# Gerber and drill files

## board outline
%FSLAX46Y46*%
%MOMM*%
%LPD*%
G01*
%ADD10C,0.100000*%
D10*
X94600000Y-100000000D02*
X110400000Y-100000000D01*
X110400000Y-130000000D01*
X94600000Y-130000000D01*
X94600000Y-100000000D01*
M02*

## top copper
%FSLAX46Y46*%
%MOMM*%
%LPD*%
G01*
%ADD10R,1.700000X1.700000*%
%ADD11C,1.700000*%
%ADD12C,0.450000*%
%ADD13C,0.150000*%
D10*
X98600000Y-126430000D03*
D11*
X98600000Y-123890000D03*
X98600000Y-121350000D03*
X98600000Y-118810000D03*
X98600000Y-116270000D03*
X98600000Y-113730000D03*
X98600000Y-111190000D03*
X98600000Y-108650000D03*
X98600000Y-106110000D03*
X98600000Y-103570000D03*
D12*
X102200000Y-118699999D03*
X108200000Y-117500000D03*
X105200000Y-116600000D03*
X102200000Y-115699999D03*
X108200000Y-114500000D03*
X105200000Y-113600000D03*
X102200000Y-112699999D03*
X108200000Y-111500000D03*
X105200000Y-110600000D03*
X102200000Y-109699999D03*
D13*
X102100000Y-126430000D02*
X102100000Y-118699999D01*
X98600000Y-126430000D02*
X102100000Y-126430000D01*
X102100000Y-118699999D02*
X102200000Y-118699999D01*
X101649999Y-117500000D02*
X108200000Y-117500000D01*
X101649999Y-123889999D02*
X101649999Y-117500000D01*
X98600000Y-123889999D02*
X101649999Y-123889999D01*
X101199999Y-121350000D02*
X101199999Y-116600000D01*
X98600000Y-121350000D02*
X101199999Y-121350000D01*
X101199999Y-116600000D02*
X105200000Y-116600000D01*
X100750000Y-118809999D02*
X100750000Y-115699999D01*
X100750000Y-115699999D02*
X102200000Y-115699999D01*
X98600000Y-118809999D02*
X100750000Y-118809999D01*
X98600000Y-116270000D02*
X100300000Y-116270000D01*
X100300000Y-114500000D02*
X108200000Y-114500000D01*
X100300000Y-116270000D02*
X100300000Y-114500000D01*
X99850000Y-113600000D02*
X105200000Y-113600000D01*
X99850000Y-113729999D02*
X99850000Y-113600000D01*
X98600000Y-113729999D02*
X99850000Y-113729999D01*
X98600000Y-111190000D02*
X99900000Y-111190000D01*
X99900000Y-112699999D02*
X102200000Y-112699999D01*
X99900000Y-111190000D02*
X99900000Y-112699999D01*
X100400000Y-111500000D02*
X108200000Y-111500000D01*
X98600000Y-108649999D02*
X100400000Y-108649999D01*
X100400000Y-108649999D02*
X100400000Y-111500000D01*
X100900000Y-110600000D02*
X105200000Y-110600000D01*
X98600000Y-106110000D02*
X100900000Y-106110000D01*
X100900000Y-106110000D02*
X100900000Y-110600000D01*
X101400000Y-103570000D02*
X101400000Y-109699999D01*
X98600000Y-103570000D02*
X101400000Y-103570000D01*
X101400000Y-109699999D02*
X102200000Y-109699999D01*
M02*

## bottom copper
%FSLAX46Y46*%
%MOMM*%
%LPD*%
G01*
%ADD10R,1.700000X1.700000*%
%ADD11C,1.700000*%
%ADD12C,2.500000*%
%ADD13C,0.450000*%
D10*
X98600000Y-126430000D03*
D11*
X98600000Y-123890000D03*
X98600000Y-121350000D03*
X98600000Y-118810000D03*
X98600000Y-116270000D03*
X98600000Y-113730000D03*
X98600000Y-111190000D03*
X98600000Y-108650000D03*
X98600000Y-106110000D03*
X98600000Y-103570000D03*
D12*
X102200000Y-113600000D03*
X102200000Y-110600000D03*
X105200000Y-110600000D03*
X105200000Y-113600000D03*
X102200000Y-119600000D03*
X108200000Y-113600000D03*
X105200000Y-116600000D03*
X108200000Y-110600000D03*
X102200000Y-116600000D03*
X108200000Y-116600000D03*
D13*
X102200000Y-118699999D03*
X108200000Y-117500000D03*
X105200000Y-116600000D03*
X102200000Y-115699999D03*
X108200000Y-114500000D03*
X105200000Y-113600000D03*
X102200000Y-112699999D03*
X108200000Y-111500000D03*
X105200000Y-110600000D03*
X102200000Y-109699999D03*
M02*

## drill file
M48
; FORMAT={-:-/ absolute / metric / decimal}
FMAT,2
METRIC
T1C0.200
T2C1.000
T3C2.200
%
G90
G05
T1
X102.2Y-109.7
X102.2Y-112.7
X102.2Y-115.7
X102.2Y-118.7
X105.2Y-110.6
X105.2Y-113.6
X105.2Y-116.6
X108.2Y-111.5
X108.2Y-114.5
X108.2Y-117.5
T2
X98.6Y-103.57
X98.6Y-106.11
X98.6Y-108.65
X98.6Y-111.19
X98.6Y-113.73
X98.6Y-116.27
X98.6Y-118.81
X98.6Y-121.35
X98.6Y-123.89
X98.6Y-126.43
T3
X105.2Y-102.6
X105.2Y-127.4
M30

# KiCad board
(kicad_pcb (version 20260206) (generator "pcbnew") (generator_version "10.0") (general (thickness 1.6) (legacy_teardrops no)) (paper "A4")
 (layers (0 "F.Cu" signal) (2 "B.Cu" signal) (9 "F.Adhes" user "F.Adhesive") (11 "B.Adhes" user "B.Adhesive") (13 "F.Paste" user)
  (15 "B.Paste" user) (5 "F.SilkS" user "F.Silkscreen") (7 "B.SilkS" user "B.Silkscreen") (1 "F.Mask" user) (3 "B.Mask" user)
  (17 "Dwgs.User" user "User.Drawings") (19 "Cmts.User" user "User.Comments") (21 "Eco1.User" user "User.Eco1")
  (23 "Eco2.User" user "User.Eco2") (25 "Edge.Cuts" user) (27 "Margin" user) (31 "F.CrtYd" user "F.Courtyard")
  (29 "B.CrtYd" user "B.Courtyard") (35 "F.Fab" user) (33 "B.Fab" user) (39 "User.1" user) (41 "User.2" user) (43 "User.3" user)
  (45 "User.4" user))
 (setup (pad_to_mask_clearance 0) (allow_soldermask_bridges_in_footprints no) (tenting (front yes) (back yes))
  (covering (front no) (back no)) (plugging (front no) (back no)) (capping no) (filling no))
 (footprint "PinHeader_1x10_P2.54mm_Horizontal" (layer "F.Cu") (at 98.6 126.43 180)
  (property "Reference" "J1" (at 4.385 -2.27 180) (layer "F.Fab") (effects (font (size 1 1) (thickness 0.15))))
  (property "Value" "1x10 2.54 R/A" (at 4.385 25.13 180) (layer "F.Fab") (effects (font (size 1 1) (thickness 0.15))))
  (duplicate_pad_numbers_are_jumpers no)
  (pad "1" thru_hole rect (at 0 0 180) (size 1.7 1.7) (drill 1) (layers "*.Cu" "*.Mask") (remove_unused_layers no) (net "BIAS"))
  (pad "2" thru_hole circle (at 0 2.54 180) (size 1.7 1.7) (drill 1) (layers "*.Cu" "*.Mask") (remove_unused_layers no) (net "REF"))
  (pad "3" thru_hole circle (at 0 5.08 180) (size 1.7 1.7) (drill 1) (layers "*.Cu" "*.Mask") (remove_unused_layers no) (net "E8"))
  (pad "4" thru_hole circle (at 0 7.62 180) (size 1.7 1.7) (drill 1) (layers "*.Cu" "*.Mask") (remove_unused_layers no) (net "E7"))
  (pad "5" thru_hole circle (at 0 10.16 180) (size 1.7 1.7) (drill 1) (layers "*.Cu" "*.Mask") (remove_unused_layers no) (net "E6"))
  (pad "6" thru_hole circle (at 0 12.7 180) (size 1.7 1.7) (drill 1) (layers "*.Cu" "*.Mask") (remove_unused_layers no) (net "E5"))
  (pad "7" thru_hole circle (at 0 15.24 180) (size 1.7 1.7) (drill 1) (layers "*.Cu" "*.Mask") (remove_unused_layers no) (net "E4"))
  (pad "8" thru_hole circle (at 0 17.78 180) (size 1.7 1.7) (drill 1) (layers "*.Cu" "*.Mask") (remove_unused_layers no) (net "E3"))
  (pad "9" thru_hole circle (at 0 20.32 180) (size 1.7 1.7) (drill 1) (layers "*.Cu" "*.Mask") (remove_unused_layers no) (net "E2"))
  (pad "10" thru_hole circle (at 0 22.86 180) (size 1.7 1.7) (drill 1) (layers "*.Cu" "*.Mask") (remove_unused_layers no) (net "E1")))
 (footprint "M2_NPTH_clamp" (layer "F.Cu") (at 105.2 102.6)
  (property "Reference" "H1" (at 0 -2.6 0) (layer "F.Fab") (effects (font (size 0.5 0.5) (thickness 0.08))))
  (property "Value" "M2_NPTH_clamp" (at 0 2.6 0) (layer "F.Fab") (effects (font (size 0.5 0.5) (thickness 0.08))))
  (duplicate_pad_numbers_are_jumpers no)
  (pad "" np_thru_hole circle (at 0 0) (size 2.2 2.2) (drill 2.2) (layers "*.Cu" "*.Mask")))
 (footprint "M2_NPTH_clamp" (layer "F.Cu") (at 105.2 127.4)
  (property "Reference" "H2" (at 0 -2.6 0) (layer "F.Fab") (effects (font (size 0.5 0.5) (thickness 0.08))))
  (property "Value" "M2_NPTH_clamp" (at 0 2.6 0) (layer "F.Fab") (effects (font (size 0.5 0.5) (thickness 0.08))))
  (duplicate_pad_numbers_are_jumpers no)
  (pad "" np_thru_hole circle (at 0 0) (size 2.2 2.2) (drill 2.2) (layers "*.Cu" "*.Mask")))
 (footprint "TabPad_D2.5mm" (layer "B.Cu") (at 102.2 113.6 180)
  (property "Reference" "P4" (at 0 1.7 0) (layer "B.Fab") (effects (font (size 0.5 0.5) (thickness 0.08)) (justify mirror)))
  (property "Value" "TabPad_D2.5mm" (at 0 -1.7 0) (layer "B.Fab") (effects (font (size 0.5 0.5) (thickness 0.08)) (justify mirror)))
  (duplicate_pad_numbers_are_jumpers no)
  (pad "1" smd circle (at 0 0 180) (size 2.5 2.5) (layers "B.Cu" "B.Mask") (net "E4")))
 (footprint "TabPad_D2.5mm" (layer "B.Cu") (at 102.2 110.6 180)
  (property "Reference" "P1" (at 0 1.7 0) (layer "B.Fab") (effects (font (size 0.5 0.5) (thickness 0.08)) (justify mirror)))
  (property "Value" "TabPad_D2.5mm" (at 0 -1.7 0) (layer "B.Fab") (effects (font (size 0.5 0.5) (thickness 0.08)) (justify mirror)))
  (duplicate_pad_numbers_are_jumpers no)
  (pad "1" smd circle (at 0 0 180) (size 2.5 2.5) (layers "B.Cu" "B.Mask") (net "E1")))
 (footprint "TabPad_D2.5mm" (layer "B.Cu") (at 105.2 110.6 180)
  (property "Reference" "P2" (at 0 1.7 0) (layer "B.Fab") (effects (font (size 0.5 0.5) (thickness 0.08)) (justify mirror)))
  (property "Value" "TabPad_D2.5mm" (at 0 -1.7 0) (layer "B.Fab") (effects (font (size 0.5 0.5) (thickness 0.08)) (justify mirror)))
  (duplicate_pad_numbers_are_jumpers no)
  (pad "1" smd circle (at 0 0 180) (size 2.5 2.5) (layers "B.Cu" "B.Mask") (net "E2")))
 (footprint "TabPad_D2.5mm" (layer "B.Cu") (at 105.2 113.6 180)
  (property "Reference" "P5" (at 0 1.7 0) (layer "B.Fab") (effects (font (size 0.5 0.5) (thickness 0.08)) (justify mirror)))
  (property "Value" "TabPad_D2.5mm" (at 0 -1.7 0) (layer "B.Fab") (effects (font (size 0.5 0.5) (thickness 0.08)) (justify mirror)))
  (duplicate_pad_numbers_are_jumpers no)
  (pad "1" smd circle (at 0 0 180) (size 2.5 2.5) (layers "B.Cu" "B.Mask") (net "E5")))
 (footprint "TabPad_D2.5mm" (layer "B.Cu") (at 102.2 119.6 180)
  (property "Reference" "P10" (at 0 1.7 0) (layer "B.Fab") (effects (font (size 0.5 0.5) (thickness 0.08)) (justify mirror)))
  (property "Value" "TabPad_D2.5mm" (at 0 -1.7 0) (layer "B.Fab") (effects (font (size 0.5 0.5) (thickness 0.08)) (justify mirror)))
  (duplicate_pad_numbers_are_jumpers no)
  (pad "1" smd circle (at 0 0 180) (size 2.5 2.5) (layers "B.Cu" "B.Mask") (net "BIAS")))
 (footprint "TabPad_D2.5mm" (layer "B.Cu") (at 108.2 113.6 180)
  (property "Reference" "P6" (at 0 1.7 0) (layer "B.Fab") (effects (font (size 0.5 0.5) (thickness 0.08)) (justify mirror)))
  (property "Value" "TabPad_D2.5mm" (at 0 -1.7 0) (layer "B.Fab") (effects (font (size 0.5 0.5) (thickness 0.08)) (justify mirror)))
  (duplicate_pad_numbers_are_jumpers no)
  (pad "1" smd circle (at 0 0 180) (size 2.5 2.5) (layers "B.Cu" "B.Mask") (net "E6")))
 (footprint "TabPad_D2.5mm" (layer "B.Cu") (at 105.2 116.6 180)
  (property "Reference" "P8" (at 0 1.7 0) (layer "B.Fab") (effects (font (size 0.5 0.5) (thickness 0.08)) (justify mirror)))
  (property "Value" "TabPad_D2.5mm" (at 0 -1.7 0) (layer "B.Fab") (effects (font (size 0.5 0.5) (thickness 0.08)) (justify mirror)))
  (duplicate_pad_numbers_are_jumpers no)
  (pad "1" smd circle (at 0 0 180) (size 2.5 2.5) (layers "B.Cu" "B.Mask") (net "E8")))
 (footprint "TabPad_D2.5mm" (layer "B.Cu") (at 108.2 110.6 180)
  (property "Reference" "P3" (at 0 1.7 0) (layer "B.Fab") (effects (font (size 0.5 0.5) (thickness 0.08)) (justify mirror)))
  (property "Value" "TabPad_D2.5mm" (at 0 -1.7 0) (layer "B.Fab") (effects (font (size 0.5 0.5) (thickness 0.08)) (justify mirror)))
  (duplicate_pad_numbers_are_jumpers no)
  (pad "1" smd circle (at 0 0 180) (size 2.5 2.5) (layers "B.Cu" "B.Mask") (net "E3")))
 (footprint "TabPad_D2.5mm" (layer "B.Cu") (at 102.2 116.6 180)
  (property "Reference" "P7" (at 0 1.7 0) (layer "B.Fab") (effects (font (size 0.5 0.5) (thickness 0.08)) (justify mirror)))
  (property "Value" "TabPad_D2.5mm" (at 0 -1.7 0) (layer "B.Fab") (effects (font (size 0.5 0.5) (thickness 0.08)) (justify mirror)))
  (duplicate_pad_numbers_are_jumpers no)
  (pad "1" smd circle (at 0 0 180) (size 2.5 2.5) (layers "B.Cu" "B.Mask") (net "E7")))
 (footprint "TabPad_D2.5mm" (layer "B.Cu") (at 108.2 116.6 180)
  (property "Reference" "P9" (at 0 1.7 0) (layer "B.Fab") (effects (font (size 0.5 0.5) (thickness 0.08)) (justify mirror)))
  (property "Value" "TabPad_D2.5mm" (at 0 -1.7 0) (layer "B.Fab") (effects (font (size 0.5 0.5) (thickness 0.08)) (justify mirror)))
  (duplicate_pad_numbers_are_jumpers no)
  (pad "1" smd circle (at 0 0 180) (size 2.5 2.5) (layers "B.Cu" "B.Mask") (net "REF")))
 (gr_rect (start 94.6 100) (end 110.4 130) (stroke (width 0.1) (type default)) (fill no) (layer "Edge.Cuts"))
 (segment (start 102.1 126.43) (end 102.1 118.699999) (width 0.15) (layer "F.Cu") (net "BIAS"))
 (segment (start 98.6 126.43) (end 102.1 126.43) (width 0.15) (layer "F.Cu") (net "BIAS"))
 (segment (start 102.1 118.699999) (end 102.2 118.699999) (width 0.15) (layer "F.Cu") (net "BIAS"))
 (via (at 102.2 118.699999) (size 0.45) (drill 0.2) (layers "F.Cu" "B.Cu") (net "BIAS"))
 (segment (start 101.649999 117.5) (end 108.2 117.5) (width 0.15) (layer "F.Cu") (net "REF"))
 (segment (start 101.649999 123.889999) (end 101.649999 117.5) (width 0.15) (layer "F.Cu") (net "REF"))
 (segment (start 98.6 123.889999) (end 101.649999 123.889999) (width 0.15) (layer "F.Cu") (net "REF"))
 (via (at 108.2 117.5) (size 0.45) (drill 0.2) (layers "F.Cu" "B.Cu") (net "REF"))
 (segment (start 101.199999 121.35) (end 101.199999 116.6) (width 0.15) (layer "F.Cu") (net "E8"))
 (segment (start 98.6 121.35) (end 101.199999 121.35) (width 0.15) (layer "F.Cu") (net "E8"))
 (segment (start 101.199999 116.6) (end 105.2 116.6) (width 0.15) (layer "F.Cu") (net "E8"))
 (via (at 105.2 116.6) (size 0.45) (drill 0.2) (layers "F.Cu" "B.Cu") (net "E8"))
 (segment (start 100.75 118.809999) (end 100.75 115.699999) (width 0.15) (layer "F.Cu") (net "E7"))
 (segment (start 100.75 115.699999) (end 102.2 115.699999) (width 0.15) (layer "F.Cu") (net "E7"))
 (segment (start 98.6 118.809999) (end 100.75 118.809999) (width 0.15) (layer "F.Cu") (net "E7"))
 (via (at 102.2 115.699999) (size 0.45) (drill 0.2) (layers "F.Cu" "B.Cu") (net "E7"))
 (segment (start 98.6 116.27) (end 100.3 116.27) (width 0.15) (layer "F.Cu") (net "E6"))
 (segment (start 100.3 114.5) (end 108.2 114.5) (width 0.15) (layer "F.Cu") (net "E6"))
 (segment (start 100.3 116.27) (end 100.3 114.5) (width 0.15) (layer "F.Cu") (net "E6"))
 (via (at 108.2 114.5) (size 0.45) (drill 0.2) (layers "F.Cu" "B.Cu") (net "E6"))
 (segment (start 99.85 113.6) (end 105.2 113.6) (width 0.15) (layer "F.Cu") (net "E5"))
 (segment (start 99.85 113.729999) (end 99.85 113.6) (width 0.15) (layer "F.Cu") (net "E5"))
 (segment (start 98.6 113.729999) (end 99.85 113.729999) (width 0.15) (layer "F.Cu") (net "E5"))
 (via (at 105.2 113.6) (size 0.45) (drill 0.2) (layers "F.Cu" "B.Cu") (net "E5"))
 (segment (start 98.6 111.19) (end 99.9 111.19) (width 0.15) (layer "F.Cu") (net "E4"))
 (segment (start 99.9 112.699999) (end 102.2 112.699999) (width 0.15) (layer "F.Cu") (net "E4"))
 (segment (start 99.9 111.19) (end 99.9 112.699999) (width 0.15) (layer "F.Cu") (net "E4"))
 (via (at 102.2 112.699999) (size 0.45) (drill 0.2) (layers "F.Cu" "B.Cu") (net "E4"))
 (segment (start 100.4 111.5) (end 108.2 111.5) (width 0.15) (layer "F.Cu") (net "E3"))
 (segment (start 98.6 108.649999) (end 100.4 108.649999) (width 0.15) (layer "F.Cu") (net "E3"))
 (segment (start 100.4 108.649999) (end 100.4 111.5) (width 0.15) (layer "F.Cu") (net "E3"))
 (via (at 108.2 111.5) (size 0.45) (drill 0.2) (layers "F.Cu" "B.Cu") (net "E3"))
 (segment (start 100.9 110.6) (end 105.2 110.6) (width 0.15) (layer "F.Cu") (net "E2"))
 (segment (start 98.6 106.11) (end 100.9 106.11) (width 0.15) (layer "F.Cu") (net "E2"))
 (segment (start 100.9 106.11) (end 100.9 110.6) (width 0.15) (layer "F.Cu") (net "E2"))
 (via (at 105.2 110.6) (size 0.45) (drill 0.2) (layers "F.Cu" "B.Cu") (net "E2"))
 (segment (start 101.4 103.57) (end 101.4 109.699999) (width 0.15) (layer "F.Cu") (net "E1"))
 (segment (start 98.6 103.57) (end 101.4 103.57) (width 0.15) (layer "F.Cu") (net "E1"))
 (segment (start 101.4 109.699999) (end 102.2 109.699999) (width 0.15) (layer "F.Cu") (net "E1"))
 (via (at 102.2 109.699999) (size 0.45) (drill 0.2) (layers "F.Cu" "B.Cu") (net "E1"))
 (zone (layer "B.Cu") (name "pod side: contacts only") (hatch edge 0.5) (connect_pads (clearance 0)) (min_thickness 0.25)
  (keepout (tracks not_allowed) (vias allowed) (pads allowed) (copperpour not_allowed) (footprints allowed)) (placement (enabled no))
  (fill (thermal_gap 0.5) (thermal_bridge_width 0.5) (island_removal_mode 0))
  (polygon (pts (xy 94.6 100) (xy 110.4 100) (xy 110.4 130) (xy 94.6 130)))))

